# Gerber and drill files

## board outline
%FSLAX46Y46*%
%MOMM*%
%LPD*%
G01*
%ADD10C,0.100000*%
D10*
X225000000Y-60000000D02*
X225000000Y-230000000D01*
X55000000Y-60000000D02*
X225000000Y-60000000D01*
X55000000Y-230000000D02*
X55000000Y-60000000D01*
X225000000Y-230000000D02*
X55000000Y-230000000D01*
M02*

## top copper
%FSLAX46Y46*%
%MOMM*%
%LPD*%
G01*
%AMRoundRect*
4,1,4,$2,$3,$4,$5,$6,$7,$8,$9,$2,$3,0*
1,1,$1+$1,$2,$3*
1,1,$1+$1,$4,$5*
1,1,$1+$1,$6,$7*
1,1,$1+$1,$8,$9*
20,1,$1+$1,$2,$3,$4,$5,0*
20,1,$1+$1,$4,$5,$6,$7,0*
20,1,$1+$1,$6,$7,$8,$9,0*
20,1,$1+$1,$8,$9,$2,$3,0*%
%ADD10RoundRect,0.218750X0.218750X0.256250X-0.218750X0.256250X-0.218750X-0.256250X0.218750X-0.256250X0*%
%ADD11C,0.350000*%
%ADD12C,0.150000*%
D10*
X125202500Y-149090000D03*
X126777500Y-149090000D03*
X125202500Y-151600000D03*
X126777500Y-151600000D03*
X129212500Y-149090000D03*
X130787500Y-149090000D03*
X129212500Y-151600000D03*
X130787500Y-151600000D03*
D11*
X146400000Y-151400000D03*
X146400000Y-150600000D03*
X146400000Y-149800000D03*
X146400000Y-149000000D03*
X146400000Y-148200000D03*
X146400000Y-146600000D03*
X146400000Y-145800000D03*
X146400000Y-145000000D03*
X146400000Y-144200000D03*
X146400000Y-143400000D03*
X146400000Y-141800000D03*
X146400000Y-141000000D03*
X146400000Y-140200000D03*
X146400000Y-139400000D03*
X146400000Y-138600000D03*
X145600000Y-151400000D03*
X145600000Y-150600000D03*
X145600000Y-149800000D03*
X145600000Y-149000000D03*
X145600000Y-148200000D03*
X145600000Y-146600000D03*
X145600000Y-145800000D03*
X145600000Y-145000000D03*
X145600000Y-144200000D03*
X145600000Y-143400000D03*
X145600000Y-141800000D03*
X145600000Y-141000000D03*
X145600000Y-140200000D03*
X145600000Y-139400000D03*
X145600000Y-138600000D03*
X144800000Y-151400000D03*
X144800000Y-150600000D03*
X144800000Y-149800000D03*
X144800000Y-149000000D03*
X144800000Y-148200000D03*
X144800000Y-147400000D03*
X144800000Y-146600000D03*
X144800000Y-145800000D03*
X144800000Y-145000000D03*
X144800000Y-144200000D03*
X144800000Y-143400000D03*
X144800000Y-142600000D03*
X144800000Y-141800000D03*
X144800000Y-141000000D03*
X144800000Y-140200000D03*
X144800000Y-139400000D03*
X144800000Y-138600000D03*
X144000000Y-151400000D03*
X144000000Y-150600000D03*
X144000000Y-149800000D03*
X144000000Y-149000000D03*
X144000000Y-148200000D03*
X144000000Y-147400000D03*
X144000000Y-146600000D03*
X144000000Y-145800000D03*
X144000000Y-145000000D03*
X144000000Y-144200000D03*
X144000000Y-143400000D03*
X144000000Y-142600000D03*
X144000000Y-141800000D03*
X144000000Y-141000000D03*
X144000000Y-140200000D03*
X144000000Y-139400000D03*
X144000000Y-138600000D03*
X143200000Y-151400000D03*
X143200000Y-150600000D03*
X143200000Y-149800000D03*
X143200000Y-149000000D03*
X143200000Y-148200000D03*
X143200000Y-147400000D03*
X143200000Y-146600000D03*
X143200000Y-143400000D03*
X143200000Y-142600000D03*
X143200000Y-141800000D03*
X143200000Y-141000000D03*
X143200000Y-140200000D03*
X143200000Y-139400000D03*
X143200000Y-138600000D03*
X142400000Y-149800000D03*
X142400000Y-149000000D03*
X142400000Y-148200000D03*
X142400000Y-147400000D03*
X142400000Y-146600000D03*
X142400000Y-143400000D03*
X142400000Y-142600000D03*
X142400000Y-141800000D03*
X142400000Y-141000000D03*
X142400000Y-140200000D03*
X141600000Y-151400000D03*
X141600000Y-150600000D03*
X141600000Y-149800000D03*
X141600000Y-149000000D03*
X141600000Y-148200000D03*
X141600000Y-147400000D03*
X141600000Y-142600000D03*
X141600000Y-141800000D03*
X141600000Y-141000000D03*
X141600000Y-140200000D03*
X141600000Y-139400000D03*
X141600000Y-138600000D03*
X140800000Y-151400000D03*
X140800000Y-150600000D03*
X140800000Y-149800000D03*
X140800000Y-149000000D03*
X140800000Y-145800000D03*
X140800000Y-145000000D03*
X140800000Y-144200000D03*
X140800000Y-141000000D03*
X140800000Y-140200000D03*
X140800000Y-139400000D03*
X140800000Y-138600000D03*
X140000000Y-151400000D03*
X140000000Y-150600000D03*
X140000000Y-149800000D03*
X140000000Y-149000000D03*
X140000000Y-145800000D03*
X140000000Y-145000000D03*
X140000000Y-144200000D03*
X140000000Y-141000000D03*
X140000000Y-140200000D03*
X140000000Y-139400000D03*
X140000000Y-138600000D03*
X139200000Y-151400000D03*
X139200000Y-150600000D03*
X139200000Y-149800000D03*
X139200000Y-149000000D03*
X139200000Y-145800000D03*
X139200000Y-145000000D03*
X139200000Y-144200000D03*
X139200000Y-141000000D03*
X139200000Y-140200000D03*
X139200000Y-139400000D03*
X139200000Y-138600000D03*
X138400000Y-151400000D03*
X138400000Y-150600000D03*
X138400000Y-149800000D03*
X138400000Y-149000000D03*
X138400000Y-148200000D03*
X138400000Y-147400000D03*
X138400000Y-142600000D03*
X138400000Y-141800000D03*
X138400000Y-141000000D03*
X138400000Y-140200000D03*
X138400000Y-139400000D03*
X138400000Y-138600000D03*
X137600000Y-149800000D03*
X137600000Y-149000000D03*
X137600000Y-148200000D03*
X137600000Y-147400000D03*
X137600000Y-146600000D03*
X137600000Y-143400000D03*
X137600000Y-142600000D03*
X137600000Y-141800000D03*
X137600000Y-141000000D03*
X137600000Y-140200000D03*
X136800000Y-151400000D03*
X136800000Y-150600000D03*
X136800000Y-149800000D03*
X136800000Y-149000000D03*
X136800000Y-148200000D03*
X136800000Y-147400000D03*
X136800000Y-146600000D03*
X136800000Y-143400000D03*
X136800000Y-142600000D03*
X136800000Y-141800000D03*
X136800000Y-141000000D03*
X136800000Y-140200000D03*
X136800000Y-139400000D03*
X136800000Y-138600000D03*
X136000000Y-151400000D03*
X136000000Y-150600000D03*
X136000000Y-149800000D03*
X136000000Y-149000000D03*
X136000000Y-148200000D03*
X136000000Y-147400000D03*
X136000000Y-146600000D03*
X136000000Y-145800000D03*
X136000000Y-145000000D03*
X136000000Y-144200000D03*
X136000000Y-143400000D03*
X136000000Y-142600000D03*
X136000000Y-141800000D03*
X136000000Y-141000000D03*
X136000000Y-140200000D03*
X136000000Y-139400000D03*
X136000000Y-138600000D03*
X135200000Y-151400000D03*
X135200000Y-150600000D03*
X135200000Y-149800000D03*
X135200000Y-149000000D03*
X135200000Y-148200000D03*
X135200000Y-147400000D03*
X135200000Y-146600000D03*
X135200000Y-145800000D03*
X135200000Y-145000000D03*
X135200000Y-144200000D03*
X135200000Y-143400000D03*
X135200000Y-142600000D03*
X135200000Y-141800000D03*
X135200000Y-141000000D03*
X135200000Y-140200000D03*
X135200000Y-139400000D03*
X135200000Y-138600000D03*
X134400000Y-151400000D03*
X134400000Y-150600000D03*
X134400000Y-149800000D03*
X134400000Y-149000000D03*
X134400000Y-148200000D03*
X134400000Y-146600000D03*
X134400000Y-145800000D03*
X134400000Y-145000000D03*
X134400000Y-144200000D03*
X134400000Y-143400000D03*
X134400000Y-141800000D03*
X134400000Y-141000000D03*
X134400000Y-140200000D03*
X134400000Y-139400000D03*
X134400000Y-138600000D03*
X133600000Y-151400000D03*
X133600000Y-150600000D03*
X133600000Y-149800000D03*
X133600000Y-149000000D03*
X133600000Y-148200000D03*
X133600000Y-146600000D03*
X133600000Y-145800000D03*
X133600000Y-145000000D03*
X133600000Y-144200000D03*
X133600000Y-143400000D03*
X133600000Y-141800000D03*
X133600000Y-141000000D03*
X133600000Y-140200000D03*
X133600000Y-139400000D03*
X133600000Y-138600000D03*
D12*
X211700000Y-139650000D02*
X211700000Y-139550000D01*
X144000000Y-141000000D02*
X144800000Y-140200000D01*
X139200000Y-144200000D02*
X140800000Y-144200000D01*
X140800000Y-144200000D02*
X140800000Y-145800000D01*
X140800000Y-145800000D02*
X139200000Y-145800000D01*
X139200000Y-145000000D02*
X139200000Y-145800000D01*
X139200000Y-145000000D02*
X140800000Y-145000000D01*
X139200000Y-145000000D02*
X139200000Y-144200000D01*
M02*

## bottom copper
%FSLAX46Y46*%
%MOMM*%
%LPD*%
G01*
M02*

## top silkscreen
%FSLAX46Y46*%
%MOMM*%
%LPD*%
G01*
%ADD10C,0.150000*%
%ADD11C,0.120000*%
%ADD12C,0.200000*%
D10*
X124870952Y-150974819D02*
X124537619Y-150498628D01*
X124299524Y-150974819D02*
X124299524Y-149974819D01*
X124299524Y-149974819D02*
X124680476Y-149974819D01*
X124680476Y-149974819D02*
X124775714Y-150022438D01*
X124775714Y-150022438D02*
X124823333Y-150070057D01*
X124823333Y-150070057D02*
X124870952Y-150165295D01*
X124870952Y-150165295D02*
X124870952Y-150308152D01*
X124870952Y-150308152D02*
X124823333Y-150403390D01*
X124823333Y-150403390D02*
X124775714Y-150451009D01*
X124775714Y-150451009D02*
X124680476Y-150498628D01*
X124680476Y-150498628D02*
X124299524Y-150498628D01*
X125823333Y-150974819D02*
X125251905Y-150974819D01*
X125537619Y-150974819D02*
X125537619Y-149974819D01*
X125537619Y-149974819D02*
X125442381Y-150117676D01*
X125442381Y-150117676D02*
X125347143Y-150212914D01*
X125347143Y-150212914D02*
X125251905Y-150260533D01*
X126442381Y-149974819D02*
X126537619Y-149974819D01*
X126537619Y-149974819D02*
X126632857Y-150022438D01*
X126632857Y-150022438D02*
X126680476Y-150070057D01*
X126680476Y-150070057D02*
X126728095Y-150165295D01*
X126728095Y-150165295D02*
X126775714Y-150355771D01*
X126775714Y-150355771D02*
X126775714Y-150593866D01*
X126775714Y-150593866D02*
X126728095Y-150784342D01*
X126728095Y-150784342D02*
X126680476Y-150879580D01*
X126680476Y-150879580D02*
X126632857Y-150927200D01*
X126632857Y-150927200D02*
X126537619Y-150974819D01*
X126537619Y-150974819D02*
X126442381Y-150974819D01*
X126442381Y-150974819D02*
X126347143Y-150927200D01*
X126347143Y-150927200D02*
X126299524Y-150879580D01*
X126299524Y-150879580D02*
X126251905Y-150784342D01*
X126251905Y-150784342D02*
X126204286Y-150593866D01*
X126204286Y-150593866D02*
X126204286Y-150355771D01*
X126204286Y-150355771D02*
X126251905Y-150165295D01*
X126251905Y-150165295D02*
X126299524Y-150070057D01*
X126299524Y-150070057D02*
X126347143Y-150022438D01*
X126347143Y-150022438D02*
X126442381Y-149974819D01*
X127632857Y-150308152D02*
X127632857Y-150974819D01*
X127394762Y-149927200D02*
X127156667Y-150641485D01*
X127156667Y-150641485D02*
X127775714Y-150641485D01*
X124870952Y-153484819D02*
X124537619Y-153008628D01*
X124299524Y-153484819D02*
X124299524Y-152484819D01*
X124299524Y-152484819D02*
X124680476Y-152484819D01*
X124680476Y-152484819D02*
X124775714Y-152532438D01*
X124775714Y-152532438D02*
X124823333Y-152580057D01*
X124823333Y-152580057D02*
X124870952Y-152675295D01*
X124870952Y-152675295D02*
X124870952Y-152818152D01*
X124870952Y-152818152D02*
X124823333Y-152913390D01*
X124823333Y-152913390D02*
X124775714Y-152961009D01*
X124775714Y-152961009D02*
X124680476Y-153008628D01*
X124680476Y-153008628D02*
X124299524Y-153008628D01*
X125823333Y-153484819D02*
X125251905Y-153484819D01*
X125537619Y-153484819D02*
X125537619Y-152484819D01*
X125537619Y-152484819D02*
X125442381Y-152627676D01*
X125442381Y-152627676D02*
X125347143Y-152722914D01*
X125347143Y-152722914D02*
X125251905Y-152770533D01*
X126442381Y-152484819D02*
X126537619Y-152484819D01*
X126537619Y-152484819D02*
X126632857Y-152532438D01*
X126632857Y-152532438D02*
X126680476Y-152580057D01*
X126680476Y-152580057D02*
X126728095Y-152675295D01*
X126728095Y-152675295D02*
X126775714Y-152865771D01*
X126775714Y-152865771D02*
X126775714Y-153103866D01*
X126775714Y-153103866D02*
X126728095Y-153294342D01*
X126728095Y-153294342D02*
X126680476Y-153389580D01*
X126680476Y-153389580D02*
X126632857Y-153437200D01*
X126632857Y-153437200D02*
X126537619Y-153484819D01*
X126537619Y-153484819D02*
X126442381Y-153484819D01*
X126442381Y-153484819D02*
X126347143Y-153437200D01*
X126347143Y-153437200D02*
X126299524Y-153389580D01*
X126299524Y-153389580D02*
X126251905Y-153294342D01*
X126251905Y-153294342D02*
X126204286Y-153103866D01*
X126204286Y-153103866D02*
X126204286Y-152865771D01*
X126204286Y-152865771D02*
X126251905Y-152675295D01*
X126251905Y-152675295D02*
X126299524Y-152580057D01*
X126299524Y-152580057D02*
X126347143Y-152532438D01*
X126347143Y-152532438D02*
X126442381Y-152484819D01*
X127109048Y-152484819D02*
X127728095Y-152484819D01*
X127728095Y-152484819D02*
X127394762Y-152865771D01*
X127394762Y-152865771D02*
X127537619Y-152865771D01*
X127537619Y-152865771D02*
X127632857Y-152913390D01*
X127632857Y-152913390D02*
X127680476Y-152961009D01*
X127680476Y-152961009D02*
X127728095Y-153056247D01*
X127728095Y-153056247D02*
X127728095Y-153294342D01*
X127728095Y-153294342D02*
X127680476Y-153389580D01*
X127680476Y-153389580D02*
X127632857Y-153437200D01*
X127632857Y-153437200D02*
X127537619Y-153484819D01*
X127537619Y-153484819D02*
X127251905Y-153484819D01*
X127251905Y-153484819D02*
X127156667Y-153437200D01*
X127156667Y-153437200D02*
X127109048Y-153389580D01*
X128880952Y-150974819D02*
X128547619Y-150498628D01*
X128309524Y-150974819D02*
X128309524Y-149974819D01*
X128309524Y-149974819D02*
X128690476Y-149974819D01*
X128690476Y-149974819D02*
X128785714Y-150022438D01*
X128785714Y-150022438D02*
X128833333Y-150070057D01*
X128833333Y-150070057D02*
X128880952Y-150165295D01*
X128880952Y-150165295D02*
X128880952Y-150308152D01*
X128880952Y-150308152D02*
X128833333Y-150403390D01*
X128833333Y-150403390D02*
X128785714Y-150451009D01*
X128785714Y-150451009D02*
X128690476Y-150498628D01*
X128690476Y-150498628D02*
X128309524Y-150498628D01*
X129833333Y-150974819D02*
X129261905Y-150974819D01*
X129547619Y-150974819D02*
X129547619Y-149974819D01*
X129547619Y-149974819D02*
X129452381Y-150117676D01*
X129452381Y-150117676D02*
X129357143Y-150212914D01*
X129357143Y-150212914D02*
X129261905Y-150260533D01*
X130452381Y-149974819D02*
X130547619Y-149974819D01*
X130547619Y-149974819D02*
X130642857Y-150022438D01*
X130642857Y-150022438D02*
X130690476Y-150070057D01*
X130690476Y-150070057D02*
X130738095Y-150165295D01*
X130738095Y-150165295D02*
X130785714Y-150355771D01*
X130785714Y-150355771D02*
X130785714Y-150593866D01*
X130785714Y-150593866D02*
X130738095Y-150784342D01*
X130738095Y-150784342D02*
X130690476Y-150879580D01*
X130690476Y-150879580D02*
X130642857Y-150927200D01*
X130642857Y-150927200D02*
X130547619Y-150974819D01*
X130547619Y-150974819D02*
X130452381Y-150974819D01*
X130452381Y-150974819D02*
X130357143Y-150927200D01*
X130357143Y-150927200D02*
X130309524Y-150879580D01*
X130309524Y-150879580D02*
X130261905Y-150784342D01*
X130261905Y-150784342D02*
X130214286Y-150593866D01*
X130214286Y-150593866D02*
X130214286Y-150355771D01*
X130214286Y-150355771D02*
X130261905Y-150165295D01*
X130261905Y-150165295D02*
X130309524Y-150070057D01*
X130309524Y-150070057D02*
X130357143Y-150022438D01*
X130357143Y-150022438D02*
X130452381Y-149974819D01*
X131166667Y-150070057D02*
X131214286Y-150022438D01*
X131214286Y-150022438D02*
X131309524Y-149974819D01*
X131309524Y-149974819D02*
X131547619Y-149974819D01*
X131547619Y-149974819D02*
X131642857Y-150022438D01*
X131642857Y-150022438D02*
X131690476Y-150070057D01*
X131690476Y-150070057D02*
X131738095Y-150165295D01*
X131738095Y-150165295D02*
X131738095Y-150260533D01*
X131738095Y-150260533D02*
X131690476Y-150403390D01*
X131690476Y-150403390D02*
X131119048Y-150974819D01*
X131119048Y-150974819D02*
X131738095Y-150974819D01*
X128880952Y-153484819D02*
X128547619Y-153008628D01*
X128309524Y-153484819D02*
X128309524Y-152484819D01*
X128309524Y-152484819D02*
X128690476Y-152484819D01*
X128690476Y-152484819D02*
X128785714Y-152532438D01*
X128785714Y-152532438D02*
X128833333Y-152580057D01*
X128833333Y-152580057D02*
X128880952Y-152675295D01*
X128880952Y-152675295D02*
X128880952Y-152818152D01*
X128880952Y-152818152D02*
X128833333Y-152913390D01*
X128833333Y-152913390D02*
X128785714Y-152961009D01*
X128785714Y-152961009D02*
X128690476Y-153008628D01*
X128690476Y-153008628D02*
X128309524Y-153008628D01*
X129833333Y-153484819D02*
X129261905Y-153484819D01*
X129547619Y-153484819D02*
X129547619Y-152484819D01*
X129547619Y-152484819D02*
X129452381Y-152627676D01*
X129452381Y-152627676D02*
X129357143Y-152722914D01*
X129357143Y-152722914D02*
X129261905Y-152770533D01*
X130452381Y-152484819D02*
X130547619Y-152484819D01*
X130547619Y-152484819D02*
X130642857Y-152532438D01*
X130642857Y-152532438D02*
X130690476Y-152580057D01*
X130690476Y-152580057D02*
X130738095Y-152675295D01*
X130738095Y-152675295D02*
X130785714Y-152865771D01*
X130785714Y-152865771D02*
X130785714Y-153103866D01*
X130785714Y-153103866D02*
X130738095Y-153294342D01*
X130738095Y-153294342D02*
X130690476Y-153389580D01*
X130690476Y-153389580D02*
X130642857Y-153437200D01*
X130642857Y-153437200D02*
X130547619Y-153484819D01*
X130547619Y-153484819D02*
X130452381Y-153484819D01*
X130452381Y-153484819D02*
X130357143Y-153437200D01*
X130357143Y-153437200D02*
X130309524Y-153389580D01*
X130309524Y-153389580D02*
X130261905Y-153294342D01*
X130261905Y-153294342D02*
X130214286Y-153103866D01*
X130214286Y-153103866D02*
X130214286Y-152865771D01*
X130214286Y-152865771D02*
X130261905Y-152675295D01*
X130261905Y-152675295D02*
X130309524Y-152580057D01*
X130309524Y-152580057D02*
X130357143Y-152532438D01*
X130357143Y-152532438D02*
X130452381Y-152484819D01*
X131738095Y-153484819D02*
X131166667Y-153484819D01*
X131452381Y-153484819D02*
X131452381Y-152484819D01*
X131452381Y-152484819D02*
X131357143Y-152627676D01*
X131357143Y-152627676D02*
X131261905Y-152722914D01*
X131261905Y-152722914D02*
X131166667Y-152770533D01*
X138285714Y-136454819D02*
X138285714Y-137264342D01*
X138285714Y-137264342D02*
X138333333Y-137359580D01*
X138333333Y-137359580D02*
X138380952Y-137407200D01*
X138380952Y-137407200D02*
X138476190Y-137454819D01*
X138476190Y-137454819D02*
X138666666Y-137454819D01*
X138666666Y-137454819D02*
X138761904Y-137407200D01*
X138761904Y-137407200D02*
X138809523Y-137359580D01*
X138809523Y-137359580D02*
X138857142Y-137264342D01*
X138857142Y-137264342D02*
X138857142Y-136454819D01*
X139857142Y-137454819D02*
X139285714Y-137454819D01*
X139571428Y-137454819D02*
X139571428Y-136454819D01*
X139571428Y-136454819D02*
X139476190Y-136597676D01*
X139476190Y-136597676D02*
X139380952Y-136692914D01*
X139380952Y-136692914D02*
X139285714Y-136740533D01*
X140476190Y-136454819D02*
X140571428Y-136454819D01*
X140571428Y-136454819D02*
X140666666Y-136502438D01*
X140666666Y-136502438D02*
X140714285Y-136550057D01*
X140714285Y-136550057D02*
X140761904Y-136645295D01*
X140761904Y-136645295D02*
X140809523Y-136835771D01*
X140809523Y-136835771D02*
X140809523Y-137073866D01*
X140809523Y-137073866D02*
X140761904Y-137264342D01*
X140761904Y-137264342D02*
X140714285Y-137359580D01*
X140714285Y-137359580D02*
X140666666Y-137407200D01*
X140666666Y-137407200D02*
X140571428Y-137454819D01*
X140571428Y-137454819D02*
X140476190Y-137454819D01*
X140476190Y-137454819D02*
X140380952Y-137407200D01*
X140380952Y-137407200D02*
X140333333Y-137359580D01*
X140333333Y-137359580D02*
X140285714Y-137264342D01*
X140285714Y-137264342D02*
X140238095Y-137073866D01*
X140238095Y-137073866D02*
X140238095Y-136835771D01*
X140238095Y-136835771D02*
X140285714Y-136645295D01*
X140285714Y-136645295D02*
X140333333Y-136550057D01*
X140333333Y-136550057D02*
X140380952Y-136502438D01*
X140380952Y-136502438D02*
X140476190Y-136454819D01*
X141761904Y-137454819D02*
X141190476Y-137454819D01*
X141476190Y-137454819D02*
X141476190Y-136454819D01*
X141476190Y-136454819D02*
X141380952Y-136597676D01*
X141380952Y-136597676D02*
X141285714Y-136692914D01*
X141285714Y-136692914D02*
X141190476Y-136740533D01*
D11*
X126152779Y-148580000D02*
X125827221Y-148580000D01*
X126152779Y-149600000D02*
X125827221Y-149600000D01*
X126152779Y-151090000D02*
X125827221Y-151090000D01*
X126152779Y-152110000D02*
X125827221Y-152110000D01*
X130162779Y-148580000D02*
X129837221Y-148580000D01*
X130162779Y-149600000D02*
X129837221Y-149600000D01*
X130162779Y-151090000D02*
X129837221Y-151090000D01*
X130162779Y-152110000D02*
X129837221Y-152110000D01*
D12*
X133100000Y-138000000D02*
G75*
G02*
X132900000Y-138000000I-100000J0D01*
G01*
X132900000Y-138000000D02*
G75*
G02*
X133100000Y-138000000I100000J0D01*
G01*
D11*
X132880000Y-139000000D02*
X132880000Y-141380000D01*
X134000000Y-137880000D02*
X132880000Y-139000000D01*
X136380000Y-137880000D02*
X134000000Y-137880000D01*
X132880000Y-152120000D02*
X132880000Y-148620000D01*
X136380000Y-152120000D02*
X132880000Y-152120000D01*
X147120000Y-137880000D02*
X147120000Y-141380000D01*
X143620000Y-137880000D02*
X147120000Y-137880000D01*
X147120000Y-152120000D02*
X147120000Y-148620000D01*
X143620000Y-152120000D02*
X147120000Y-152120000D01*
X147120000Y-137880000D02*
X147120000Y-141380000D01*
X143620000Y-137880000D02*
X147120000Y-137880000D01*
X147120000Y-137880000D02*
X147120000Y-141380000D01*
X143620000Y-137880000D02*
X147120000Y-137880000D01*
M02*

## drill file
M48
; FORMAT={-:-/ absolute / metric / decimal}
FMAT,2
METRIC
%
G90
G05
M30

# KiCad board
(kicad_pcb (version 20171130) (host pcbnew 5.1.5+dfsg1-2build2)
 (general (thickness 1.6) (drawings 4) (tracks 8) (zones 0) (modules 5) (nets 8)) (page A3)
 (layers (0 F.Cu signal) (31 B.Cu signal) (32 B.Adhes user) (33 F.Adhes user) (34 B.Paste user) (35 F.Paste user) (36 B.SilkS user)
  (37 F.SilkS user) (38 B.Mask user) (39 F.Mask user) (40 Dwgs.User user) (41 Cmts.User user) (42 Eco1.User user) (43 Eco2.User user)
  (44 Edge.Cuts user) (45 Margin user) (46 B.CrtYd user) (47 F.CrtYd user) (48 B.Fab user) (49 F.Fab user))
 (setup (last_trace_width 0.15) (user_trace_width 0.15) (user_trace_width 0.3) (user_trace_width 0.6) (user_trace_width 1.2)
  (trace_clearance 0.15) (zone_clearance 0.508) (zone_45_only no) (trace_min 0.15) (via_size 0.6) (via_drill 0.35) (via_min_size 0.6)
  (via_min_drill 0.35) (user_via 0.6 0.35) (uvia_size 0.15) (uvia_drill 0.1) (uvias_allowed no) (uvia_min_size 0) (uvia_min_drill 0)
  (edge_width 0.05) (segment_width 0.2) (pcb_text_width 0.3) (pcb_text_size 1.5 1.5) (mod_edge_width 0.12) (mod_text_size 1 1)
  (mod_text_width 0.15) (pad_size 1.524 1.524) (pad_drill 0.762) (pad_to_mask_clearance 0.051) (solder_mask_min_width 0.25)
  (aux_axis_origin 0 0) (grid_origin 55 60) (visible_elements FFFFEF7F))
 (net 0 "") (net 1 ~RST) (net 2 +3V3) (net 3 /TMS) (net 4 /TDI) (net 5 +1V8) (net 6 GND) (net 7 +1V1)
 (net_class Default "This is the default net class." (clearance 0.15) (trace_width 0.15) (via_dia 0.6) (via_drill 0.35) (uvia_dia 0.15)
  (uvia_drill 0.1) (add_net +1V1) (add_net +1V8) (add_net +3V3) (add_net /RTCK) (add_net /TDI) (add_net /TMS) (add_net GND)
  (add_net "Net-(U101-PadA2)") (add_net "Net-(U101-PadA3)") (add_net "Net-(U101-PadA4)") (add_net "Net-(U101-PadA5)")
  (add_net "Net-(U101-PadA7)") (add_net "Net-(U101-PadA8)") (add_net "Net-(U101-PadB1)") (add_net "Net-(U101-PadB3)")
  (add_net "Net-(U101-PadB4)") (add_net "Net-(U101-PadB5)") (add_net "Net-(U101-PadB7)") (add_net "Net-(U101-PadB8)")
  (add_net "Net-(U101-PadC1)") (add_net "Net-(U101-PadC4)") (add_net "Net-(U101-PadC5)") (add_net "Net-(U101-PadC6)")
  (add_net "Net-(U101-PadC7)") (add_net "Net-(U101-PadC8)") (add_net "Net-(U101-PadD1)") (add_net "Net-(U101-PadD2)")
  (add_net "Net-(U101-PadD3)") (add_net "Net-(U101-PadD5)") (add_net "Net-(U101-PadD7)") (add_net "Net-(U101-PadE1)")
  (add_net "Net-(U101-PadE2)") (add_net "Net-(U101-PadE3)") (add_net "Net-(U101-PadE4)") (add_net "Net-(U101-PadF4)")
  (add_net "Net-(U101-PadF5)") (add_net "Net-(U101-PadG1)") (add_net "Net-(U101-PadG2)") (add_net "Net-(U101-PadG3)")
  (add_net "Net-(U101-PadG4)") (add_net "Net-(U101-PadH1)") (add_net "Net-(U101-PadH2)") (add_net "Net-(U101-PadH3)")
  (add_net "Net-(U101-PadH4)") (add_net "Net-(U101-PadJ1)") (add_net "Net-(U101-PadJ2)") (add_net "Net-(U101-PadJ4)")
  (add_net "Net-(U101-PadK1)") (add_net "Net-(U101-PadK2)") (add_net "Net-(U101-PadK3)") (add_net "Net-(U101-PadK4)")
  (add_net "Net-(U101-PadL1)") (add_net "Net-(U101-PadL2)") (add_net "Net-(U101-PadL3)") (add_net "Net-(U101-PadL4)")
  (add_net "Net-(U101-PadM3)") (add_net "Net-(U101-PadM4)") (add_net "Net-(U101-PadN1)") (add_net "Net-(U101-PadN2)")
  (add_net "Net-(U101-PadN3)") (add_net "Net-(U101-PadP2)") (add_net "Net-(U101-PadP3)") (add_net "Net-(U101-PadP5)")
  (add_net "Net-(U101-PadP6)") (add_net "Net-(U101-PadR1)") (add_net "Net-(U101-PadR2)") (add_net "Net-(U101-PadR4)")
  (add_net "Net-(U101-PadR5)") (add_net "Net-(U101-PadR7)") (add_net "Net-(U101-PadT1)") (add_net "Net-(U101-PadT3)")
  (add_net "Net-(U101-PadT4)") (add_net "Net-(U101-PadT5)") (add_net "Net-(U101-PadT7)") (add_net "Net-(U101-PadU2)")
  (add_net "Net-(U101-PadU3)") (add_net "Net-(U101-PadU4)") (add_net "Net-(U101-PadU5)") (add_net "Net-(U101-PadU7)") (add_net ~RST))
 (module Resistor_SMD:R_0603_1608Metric (layer F.Cu) (at 125.99 149.09 180)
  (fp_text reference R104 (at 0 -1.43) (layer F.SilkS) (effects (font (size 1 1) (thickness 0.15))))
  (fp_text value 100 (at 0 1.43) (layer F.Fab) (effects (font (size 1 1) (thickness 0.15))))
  (fp_line (start -0.162779 0.51) (end 0.162779 0.51) (layer F.SilkS) (width 0.12))
  (fp_line (start -0.162779 -0.51) (end 0.162779 -0.51) (layer F.SilkS) (width 0.12))
  (pad 2 smd roundrect (at 0.7875 0 180) (size 0.875 0.95) (layers F.Cu F.Paste F.Mask) (roundrect_rratio 0.25))
  (pad 1 smd roundrect (at -0.7875 0 180) (size 0.875 0.95) (layers F.Cu F.Paste F.Mask) (roundrect_rratio 0.25) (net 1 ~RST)))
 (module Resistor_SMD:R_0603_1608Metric (layer F.Cu) (at 125.99 151.6 180)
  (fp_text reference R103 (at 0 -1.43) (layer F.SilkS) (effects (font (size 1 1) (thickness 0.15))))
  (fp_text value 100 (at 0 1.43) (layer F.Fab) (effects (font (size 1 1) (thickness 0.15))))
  (fp_line (start -0.162779 0.51) (end 0.162779 0.51) (layer F.SilkS) (width 0.12))
  (fp_line (start -0.162779 -0.51) (end 0.162779 -0.51) (layer F.SilkS) (width 0.12))
  (pad 2 smd roundrect (at 0.7875 0 180) (size 0.875 0.95) (layers F.Cu F.Paste F.Mask) (roundrect_rratio 0.25) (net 1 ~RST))
  (pad 1 smd roundrect (at -0.7875 0 180) (size 0.875 0.95) (layers F.Cu F.Paste F.Mask) (roundrect_rratio 0.25) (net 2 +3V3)))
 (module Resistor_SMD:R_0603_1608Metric (layer F.Cu) (at 130 149.09 180)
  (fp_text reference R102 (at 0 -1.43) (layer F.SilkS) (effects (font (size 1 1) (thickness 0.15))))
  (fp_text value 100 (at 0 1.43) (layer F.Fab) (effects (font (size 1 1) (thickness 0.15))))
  (fp_line (start -0.162779 0.51) (end 0.162779 0.51) (layer F.SilkS) (width 0.12))
  (fp_line (start -0.162779 -0.51) (end 0.162779 -0.51) (layer F.SilkS) (width 0.12))
  (pad 2 smd roundrect (at 0.7875 0 180) (size 0.875 0.95) (layers F.Cu F.Paste F.Mask) (roundrect_rratio 0.25) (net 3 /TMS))
  (pad 1 smd roundrect (at -0.7875 0 180) (size 0.875 0.95) (layers F.Cu F.Paste F.Mask) (roundrect_rratio 0.25) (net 2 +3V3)))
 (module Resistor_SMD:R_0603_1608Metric (layer F.Cu) (at 130 151.6 180)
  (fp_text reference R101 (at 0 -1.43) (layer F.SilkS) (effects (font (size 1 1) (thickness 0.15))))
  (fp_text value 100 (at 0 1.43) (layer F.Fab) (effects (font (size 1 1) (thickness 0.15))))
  (fp_line (start -0.162779 0.51) (end 0.162779 0.51) (layer F.SilkS) (width 0.12))
  (fp_line (start -0.162779 -0.51) (end 0.162779 -0.51) (layer F.SilkS) (width 0.12))
  (pad 2 smd roundrect (at 0.7875 0 180) (size 0.875 0.95) (layers F.Cu F.Paste F.Mask) (roundrect_rratio 0.25) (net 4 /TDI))
  (pad 1 smd roundrect (at -0.7875 0 180) (size 0.875 0.95) (layers F.Cu F.Paste F.Mask) (roundrect_rratio 0.25) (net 2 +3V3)))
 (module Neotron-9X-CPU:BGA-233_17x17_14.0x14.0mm (layer F.Cu) (at 140 145)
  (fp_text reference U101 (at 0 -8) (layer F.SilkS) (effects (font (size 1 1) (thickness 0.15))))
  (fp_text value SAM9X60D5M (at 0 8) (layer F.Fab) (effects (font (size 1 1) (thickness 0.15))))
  (fp_circle (center -7 -7) (end -7 -6.9) (layer F.SilkS) (width 0.2))
  (fp_line (start -7.12 -6) (end -7.12 -3.62) (layer F.SilkS) (width 0.12))
  (fp_line (start -6 -7.12) (end -7.12 -6) (layer F.SilkS) (width 0.12))
  (fp_line (start -3.62 -7.12) (end -6 -7.12) (layer F.SilkS) (width 0.12))
  (fp_line (start -7.12 7.12) (end -7.12 3.62) (layer F.SilkS) (width 0.12))
  (fp_line (start -3.62 7.12) (end -7.12 7.12) (layer F.SilkS) (width 0.12))
  (fp_line (start 7.12 -7.12) (end 7.12 -3.62) (layer F.SilkS) (width 0.12))
  (fp_line (start 3.62 -7.12) (end 7.12 -7.12) (layer F.SilkS) (width 0.12))
  (fp_line (start 7.12 7.12) (end 7.12 3.62) (layer F.SilkS) (width 0.12))
  (fp_line (start 3.62 7.12) (end 7.12 7.12) (layer F.SilkS) (width 0.12))
  (fp_line (start 7.12 -7.12) (end 7.12 -3.62) (layer F.SilkS) (width 0.12))
  (fp_line (start 3.62 -7.12) (end 7.12 -7.12) (layer F.SilkS) (width 0.12))
  (fp_line (start 7.12 -7.12) (end 7.12 -3.62) (layer F.SilkS) (width 0.12))
  (fp_line (start 3.62 -7.12) (end 7.12 -7.12) (layer F.SilkS) (width 0.12))
  (pad U17 smd circle (at 6.4 6.4) (size 0.35 0.35) (layers F.Cu F.Paste F.Mask))
  (pad T17 smd circle (at 6.4 5.6) (size 0.35 0.35) (layers F.Cu F.Paste F.Mask))
  (pad R17 smd circle (at 6.4 4.8) (size 0.35 0.35) (layers F.Cu F.Paste F.Mask))
  (pad P17 smd circle (at 6.4 4) (size 0.35 0.35) (layers F.Cu F.Paste F.Mask))
  (pad N17 smd circle (at 6.4 3.2) (size 0.35 0.35) (layers F.Cu F.Paste F.Mask))
  (pad L17 smd circle (at 6.4 1.6) (size 0.35 0.35) (layers F.Cu F.Paste F.Mask))
  (pad K17 smd circle (at 6.4 0.8) (size 0.35 0.35) (layers F.Cu F.Paste F.Mask))
  (pad J17 smd circle (at 6.4 0) (size 0.35 0.35) (layers F.Cu F.Paste F.Mask))
  (pad H17 smd circle (at 6.4 -0.8) (size 0.35 0.35) (layers F.Cu F.Paste F.Mask))
  (pad G17 smd circle (at 6.4 -1.6) (size 0.35 0.35) (layers F.Cu F.Paste F.Mask))
  (pad E17 smd circle (at 6.4 -3.2) (size 0.35 0.35) (layers F.Cu F.Paste F.Mask))
  (pad D17 smd circle (at 6.4 -4) (size 0.35 0.35) (layers F.Cu F.Paste F.Mask))
  (pad C17 smd circle (at 6.4 -4.8) (size 0.35 0.35) (layers F.Cu F.Paste F.Mask))
  (pad B17 smd circle (at 6.4 -5.6) (size 0.35 0.35) (layers F.Cu F.Paste F.Mask) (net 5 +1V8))
  (pad A17 smd circle (at 6.4 -6.4) (size 0.35 0.35) (layers F.Cu F.Paste F.Mask) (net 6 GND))
  (pad U16 smd circle (at 5.6 6.4) (size 0.35 0.35) (layers F.Cu F.Paste F.Mask))
  (pad T16 smd circle (at 5.6 5.6) (size 0.35 0.35) (layers F.Cu F.Paste F.Mask) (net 6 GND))
  (pad R16 smd circle (at 5.6 4.8) (size 0.35 0.35) (layers F.Cu F.Paste F.Mask) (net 6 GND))
  (pad P16 smd circle (at 5.6 4) (size 0.35 0.35) (layers F.Cu F.Paste F.Mask))
  (pad N16 smd circle (at 5.6 3.2) (size 0.35 0.35) (layers F.Cu F.Paste F.Mask) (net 3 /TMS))
  (pad L16 smd circle (at 5.6 1.6) (size 0.35 0.35) (layers F.Cu F.Paste F.Mask))
  (pad K16 smd circle (at 5.6 0.8) (size 0.35 0.35) (layers F.Cu F.Paste F.Mask))
  (pad J16 smd circle (at 5.6 0) (size 0.35 0.35) (layers F.Cu F.Paste F.Mask))
  (pad H16 smd circle (at 5.6 -0.8) (size 0.35 0.35) (layers F.Cu F.Paste F.Mask))
  (pad G16 smd circle (at 5.6 -1.6) (size 0.35 0.35) (layers F.Cu F.Paste F.Mask))
  (pad E16 smd circle (at 5.6 -3.2) (size 0.35 0.35) (layers F.Cu F.Paste F.Mask))
  (pad D16 smd circle (at 5.6 -4) (size 0.35 0.35) (layers F.Cu F.Paste F.Mask))
  (pad C16 smd circle (at 5.6 -4.8) (size 0.35 0.35) (layers F.Cu F.Paste F.Mask) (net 5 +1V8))
  (pad B16 smd circle (at 5.6 -5.6) (size 0.35 0.35) (layers F.Cu F.Paste F.Mask) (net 6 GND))
  (pad A16 smd circle (at 5.6 -6.4) (size 0.35 0.35) (layers F.Cu F.Paste F.Mask) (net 5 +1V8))
  (pad U15 smd circle (at 4.8 6.4) (size 0.35 0.35) (layers F.Cu F.Paste F.Mask) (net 6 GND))
  (pad T15 smd circle (at 4.8 5.6) (size 0.35 0.35) (layers F.Cu F.Paste F.Mask))
  (pad R15 smd circle (at 4.8 4.8) (size 0.35 0.35) (layers F.Cu F.Paste F.Mask) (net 6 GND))
  (pad P15 smd circle (at 4.8 4) (size 0.35 0.35) (layers F.Cu F.Paste F.Mask))
  (pad N15 smd circle (at 4.8 3.2) (size 0.35 0.35) (layers F.Cu F.Paste F.Mask))
  (pad M15 smd circle (at 4.8 2.4) (size 0.35 0.35) (layers F.Cu F.Paste F.Mask))
  (pad L15 smd circle (at 4.8 1.6) (size 0.35 0.35) (layers F.Cu F.Paste F.Mask) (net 4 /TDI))
  (pad K15 smd circle (at 4.8 0.8) (size 0.35 0.35) (layers F.Cu F.Paste F.Mask))
  (pad J15 smd circle (at 4.8 0) (size 0.35 0.35) (layers F.Cu F.Paste F.Mask) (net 6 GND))
  (pad H15 smd circle (at 4.8 -0.8) (size 0.35 0.35) (layers F.Cu F.Paste F.Mask))
  (pad G15 smd circle (at 4.8 -1.6) (size 0.35 0.35) (layers F.Cu F.Paste F.Mask))
  (pad F15 smd circle (at 4.8 -2.4) (size 0.35 0.35) (layers F.Cu F.Paste F.Mask) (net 6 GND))
  (pad E15 smd circle (at 4.8 -3.2) (size 0.35 0.35) (layers F.Cu F.Paste F.Mask))
  (pad D15 smd circle (at 4.8 -4) (size 0.35 0.35) (layers F.Cu F.Paste F.Mask) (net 5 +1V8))
  (pad C15 smd circle (at 4.8 -4.8) (size 0.35 0.35) (layers F.Cu F.Paste F.Mask) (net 6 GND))
  (pad B15 smd circle (at 4.8 -5.6) (size 0.35 0.35) (layers F.Cu F.Paste F.Mask) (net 5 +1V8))
  (pad A15 smd circle (at 4.8 -6.4) (size 0.35 0.35) (layers F.Cu F.Paste F.Mask) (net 6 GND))
  (pad U14 smd circle (at 4 6.4) (size 0.35 0.35) (layers F.Cu F.Paste F.Mask))
  (pad T14 smd circle (at 4 5.6) (size 0.35 0.35) (layers F.Cu F.Paste F.Mask))
  (pad R14 smd circle (at 4 4.8) (size 0.35 0.35) (layers F.Cu F.Paste F.Mask))
  (pad P14 smd circle (at 4 4) (size 0.35 0.35) (layers F.Cu F.Paste F.Mask) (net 6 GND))
  (pad N14 smd circle (at 4 3.2) (size 0.35 0.35) (layers F.Cu F.Paste F.Mask))
  (pad M14 smd circle (at 4 2.4) (size 0.35 0.35) (layers F.Cu F.Paste F.Mask) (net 6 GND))
  (pad L14 smd circle (at 4 1.6) (size 0.35 0.35) (layers F.Cu F.Paste F.Mask) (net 6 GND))
  (pad K14 smd circle (at 4 0.8) (size 0.35 0.35) (layers F.Cu F.Paste F.Mask))
  (pad J14 smd circle (at 4 0) (size 0.35 0.35) (layers F.Cu F.Paste F.Mask))
  (pad H14 smd circle (at 4 -0.8) (size 0.35 0.35) (layers F.Cu F.Paste F.Mask))
  (pad G14 smd circle (at 4 -1.6) (size 0.35 0.35) (layers F.Cu F.Paste F.Mask))
  (pad F14 smd circle (at 4 -2.4) (size 0.35 0.35) (layers F.Cu F.Paste F.Mask))
  (pad E14 smd circle (at 4 -3.2) (size 0.35 0.35) (layers F.Cu F.Paste F.Mask))
  (pad D14 smd circle (at 4 -4) (size 0.35 0.35) (layers F.Cu F.Paste F.Mask) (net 6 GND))
  (pad C14 smd circle (at 4 -4.8) (size 0.35 0.35) (layers F.Cu F.Paste F.Mask) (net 5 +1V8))
  (pad B14 smd circle (at 4 -5.6) (size 0.35 0.35) (layers F.Cu F.Paste F.Mask) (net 6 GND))
  (pad A14 smd circle (at 4 -6.4) (size 0.35 0.35) (layers F.Cu F.Paste F.Mask))
  (pad U13 smd circle (at 3.2 6.4) (size 0.35 0.35) (layers F.Cu F.Paste F.Mask))
  (pad T13 smd circle (at 3.2 5.6) (size 0.35 0.35) (layers F.Cu F.Paste F.Mask))
  (pad R13 smd circle (at 3.2 4.8) (size 0.35 0.35) (layers F.Cu F.Paste F.Mask))
  (pad P13 smd circle (at 3.2 4) (size 0.35 0.35) (layers F.Cu F.Paste F.Mask))
  (pad N13 smd circle (at 3.2 3.2) (size 0.35 0.35) (layers F.Cu F.Paste F.Mask) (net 6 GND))
  (pad M13 smd circle (at 3.2 2.4) (size 0.35 0.35) (layers F.Cu F.Paste F.Mask) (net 6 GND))
  (pad L13 smd circle (at 3.2 1.6) (size 0.35 0.35) (layers F.Cu F.Paste F.Mask) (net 6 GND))
  (pad G13 smd circle (at 3.2 -1.6) (size 0.35 0.35) (layers F.Cu F.Paste F.Mask) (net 5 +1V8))
  (pad F13 smd circle (at 3.2 -2.4) (size 0.35 0.35) (layers F.Cu F.Paste F.Mask) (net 5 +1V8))
  (pad E13 smd circle (at 3.2 -3.2) (size 0.35 0.35) (layers F.Cu F.Paste F.Mask) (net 6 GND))
  (pad D13 smd circle (at 3.2 -4) (size 0.35 0.35) (layers F.Cu F.Paste F.Mask) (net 5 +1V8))
  (pad C13 smd circle (at 3.2 -4.8) (size 0.35 0.35) (layers F.Cu F.Paste F.Mask) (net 6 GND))
  (pad B13 smd circle (at 3.2 -5.6) (size 0.35 0.35) (layers F.Cu F.Paste F.Mask) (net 6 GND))
  (pad A13 smd circle (at 3.2 -6.4) (size 0.35 0.35) (layers F.Cu F.Paste F.Mask) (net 6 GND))
  (pad R12 smd circle (at 2.4 4.8) (size 0.35 0.35) (layers F.Cu F.Paste F.Mask))
  (pad P12 smd circle (at 2.4 4) (size 0.35 0.35) (layers F.Cu F.Paste F.Mask))
  (pad N12 smd circle (at 2.4 3.2) (size 0.35 0.35) (layers F.Cu F.Paste F.Mask) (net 6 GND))
  (pad M12 smd circle (at 2.4 2.4) (size 0.35 0.35) (layers F.Cu F.Paste F.Mask) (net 6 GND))
  (pad L12 smd circle (at 2.4 1.6) (size 0.35 0.35) (layers F.Cu F.Paste F.Mask) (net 6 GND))
  (pad G12 smd circle (at 2.4 -1.6) (size 0.35 0.35) (layers F.Cu F.Paste F.Mask) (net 6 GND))
  (pad F12 smd circle (at 2.4 -2.4) (size 0.35 0.35) (layers F.Cu F.Paste F.Mask) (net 6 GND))
  (pad E12 smd circle (at 2.4 -3.2) (size 0.35 0.35) (layers F.Cu F.Paste F.Mask) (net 5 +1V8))
  (pad D12 smd circle (at 2.4 -4) (size 0.35 0.35) (layers F.Cu F.Paste F.Mask))
  (pad C12 smd circle (at 2.4 -4.8) (size 0.35 0.35) (layers F.Cu F.Paste F.Mask) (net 6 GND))
  (pad U11 smd circle (at 1.6 6.4) (size 0.35 0.35) (layers F.Cu F.Paste F.Mask))
  (pad T11 smd circle (at 1.6 5.6) (size 0.35 0.35) (layers F.Cu F.Paste F.Mask))
  (pad R11 smd circle (at 1.6 4.8) (size 0.35 0.35) (layers F.Cu F.Paste F.Mask) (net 6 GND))
  (pad P11 smd circle (at 1.6 4) (size 0.35 0.35) (layers F.Cu F.Paste F.Mask))
  (pad N11 smd circle (at 1.6 3.2) (size 0.35 0.35) (layers F.Cu F.Paste F.Mask))
  (pad M11 smd circle (at 1.6 2.4) (size 0.35 0.35) (layers F.Cu F.Paste F.Mask) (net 6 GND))
  (pad F11 smd circle (at 1.6 -2.4) (size 0.35 0.35) (layers F.Cu F.Paste F.Mask) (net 6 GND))
  (pad E11 smd circle (at 1.6 -3.2) (size 0.35 0.35) (layers F.Cu F.Paste F.Mask) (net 5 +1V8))
  (pad D11 smd circle (at 1.6 -4) (size 0.35 0.35) (layers F.Cu F.Paste F.Mask))
  (pad C11 smd circle (at 1.6 -4.8) (size 0.35 0.35) (layers F.Cu F.Paste F.Mask))
  (pad B11 smd circle (at 1.6 -5.6) (size 0.35 0.35) (layers F.Cu F.Paste F.Mask))
  (pad A11 smd circle (at 1.6 -6.4) (size 0.35 0.35) (layers F.Cu F.Paste F.Mask))
  (pad U10 smd circle (at 0.8 6.4) (size 0.35 0.35) (layers F.Cu F.Paste F.Mask))
  (pad T10 smd circle (at 0.8 5.6) (size 0.35 0.35) (layers F.Cu F.Paste F.Mask))
  (pad R10 smd circle (at 0.8 4.8) (size 0.35 0.35) (layers F.Cu F.Paste F.Mask))
  (pad P10 smd circle (at 0.8 4) (size 0.35 0.35) (layers F.Cu F.Paste F.Mask) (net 6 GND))
  (pad K10 smd circle (at 0.8 0.8) (size 0.35 0.35) (layers F.Cu F.Paste F.Mask) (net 6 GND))
  (pad J10 smd circle (at 0.8 0) (size 0.35 0.35) (layers F.Cu F.Paste F.Mask) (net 6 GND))
  (pad H10 smd circle (at 0.8 -0.8) (size 0.35 0.35) (layers F.Cu F.Paste F.Mask) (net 6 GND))
  (pad D10 smd circle (at 0.8 -4) (size 0.35 0.35) (layers F.Cu F.Paste F.Mask))
  (pad C10 smd circle (at 0.8 -4.8) (size 0.35 0.35) (layers F.Cu F.Paste F.Mask))
  (pad B10 smd circle (at 0.8 -5.6) (size 0.35 0.35) (layers F.Cu F.Paste F.Mask))
  (pad A10 smd circle (at 0.8 -6.4) (size 0.35 0.35) (layers F.Cu F.Paste F.Mask))
  (pad U9 smd circle (at 0 6.4) (size 0.35 0.35) (layers F.Cu F.Paste F.Mask))
  (pad T9 smd circle (at 0 5.6) (size 0.35 0.35) (layers F.Cu F.Paste F.Mask))
  (pad R9 smd circle (at 0 4.8) (size 0.35 0.35) (layers F.Cu F.Paste F.Mask) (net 6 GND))
  (pad P9 smd circle (at 0 4) (size 0.35 0.35) (layers F.Cu F.Paste F.Mask))
  (pad K9 smd circle (at 0 0.8) (size 0.35 0.35) (layers F.Cu F.Paste F.Mask) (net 6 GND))
  (pad J9 smd circle (at 0 0) (size 0.35 0.35) (layers F.Cu F.Paste F.Mask) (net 6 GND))
  (pad H9 smd circle (at 0 -0.8) (size 0.35 0.35) (layers F.Cu F.Paste F.Mask) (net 6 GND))
  (pad D9 smd circle (at 0 -4) (size 0.35 0.35) (layers F.Cu F.Paste F.Mask))
  (pad C9 smd circle (at 0 -4.8) (size 0.35 0.35) (layers F.Cu F.Paste F.Mask) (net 6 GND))
  (pad B9 smd circle (at 0 -5.6) (size 0.35 0.35) (layers F.Cu F.Paste F.Mask))
  (pad A9 smd circle (at 0 -6.4) (size 0.35 0.35) (layers F.Cu F.Paste F.Mask))
  (pad U8 smd circle (at -0.8 6.4) (size 0.35 0.35) (layers F.Cu F.Paste F.Mask))
  (pad T8 smd circle (at -0.8 5.6) (size 0.35 0.35) (layers F.Cu F.Paste F.Mask))
  (pad R8 smd circle (at -0.8 4.8) (size 0.35 0.35) (layers F.Cu F.Paste F.Mask))
  (pad P8 smd circle (at -0.8 4) (size 0.35 0.35) (layers F.Cu F.Paste F.Mask))
  (pad K8 smd circle (at -0.8 0.8) (size 0.35 0.35) (layers F.Cu F.Paste F.Mask) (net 6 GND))
  (pad J8 smd circle (at -0.8 0) (size 0.35 0.35) (layers F.Cu F.Paste F.Mask) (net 6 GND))
  (pad H8 smd circle (at -0.8 -0.8) (size 0.35 0.35) (layers F.Cu F.Paste F.Mask) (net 6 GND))
  (pad D8 smd circle (at -0.8 -4) (size 0.35 0.35) (layers F.Cu F.Paste F.Mask) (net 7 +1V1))
  (pad C8 smd circle (at -0.8 -4.8) (size 0.35 0.35) (layers F.Cu F.Paste F.Mask))
  (pad B8 smd circle (at -0.8 -5.6) (size 0.35 0.35) (layers F.Cu F.Paste F.Mask))
  (pad A8 smd circle (at -0.8 -6.4) (size 0.35 0.35) (layers F.Cu F.Paste F.Mask))
  (pad U7 smd circle (at -1.6 6.4) (size 0.35 0.35) (layers F.Cu F.Paste F.Mask))
  (pad T7 smd circle (at -1.6 5.6) (size 0.35 0.35) (layers F.Cu F.Paste F.Mask))
  (pad R7 smd circle (at -1.6 4.8) (size 0.35 0.35) (layers F.Cu F.Paste F.Mask))
  (pad P7 smd circle (at -1.6 4) (size 0.35 0.35) (layers F.Cu F.Paste F.Mask) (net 6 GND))
  (pad N7 smd circle (at -1.6 3.2) (size 0.35 0.35) (layers F.Cu F.Paste F.Mask) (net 6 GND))
  (pad M7 smd circle (at -1.6 2.4) (size 0.35 0.35) (layers F.Cu F.Paste F.Mask) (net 7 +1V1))
  (pad F7 smd circle (at -1.6 -2.4) (size 0.35 0.35) (layers F.Cu F.Paste F.Mask) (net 6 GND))
  (pad E7 smd circle (at -1.6 -3.2) (size 0.35 0.35) (layers F.Cu F.Paste F.Mask) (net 6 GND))
  (pad D7 smd circle (at -1.6 -4) (size 0.35 0.35) (layers F.Cu F.Paste F.Mask))
  (pad C7 smd circle (at -1.6 -4.8) (size 0.35 0.35) (layers F.Cu F.Paste F.Mask))
  (pad B7 smd circle (at -1.6 -5.6) (size 0.35 0.35) (layers F.Cu F.Paste F.Mask))
  (pad A7 smd circle (at -1.6 -6.4) (size 0.35 0.35) (layers F.Cu F.Paste F.Mask))
  (pad R6 smd circle (at -2.4 4.8) (size 0.35 0.35) (layers F.Cu F.Paste F.Mask) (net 7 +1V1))
  (pad P6 smd circle (at -2.4 4) (size 0.35 0.35) (layers F.Cu F.Paste F.Mask))
  (pad N6 smd circle (at -2.4 3.2) (size 0.35 0.35) (layers F.Cu F.Paste F.Mask) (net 6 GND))
  (pad M6 smd circle (at -2.4 2.4) (size 0.35 0.35) (layers F.Cu F.Paste F.Mask) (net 6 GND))
  (pad L6 smd circle (at -2.4 1.6) (size 0.35 0.35) (layers F.Cu F.Paste F.Mask) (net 7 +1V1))
  (pad G6 smd circle (at -2.4 -1.6) (size 0.35 0.35) (layers F.Cu F.Paste F.Mask) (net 6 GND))
  (pad F6 smd circle (at -2.4 -2.4) (size 0.35 0.35) (layers F.Cu F.Paste F.Mask) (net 6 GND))
  (pad E6 smd circle (at -2.4 -3.2) (size 0.35 0.35) (layers F.Cu F.Paste F.Mask) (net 6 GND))
  (pad D6 smd circle (at -2.4 -4) (size 0.35 0.35) (layers F.Cu F.Paste F.Mask) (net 7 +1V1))
  (pad C6 smd circle (at -2.4 -4.8) (size 0.35 0.35) (layers F.Cu F.Paste F.Mask))
  (pad U5 smd circle (at -3.2 6.4) (size 0.35 0.35) (layers F.Cu F.Paste F.Mask))
  (pad T5 smd circle (at -3.2 5.6) (size 0.35 0.35) (layers F.Cu F.Paste F.Mask))
  (pad R5 smd circle (at -3.2 4.8) (size 0.35 0.35) (layers F.Cu F.Paste F.Mask))
  (pad P5 smd circle (at -3.2 4) (size 0.35 0.35) (layers F.Cu F.Paste F.Mask))
  (pad N5 smd circle (at -3.2 3.2) (size 0.35 0.35) (layers F.Cu F.Paste F.Mask) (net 6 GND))
  (pad M5 smd circle (at -3.2 2.4) (size 0.35 0.35) (layers F.Cu F.Paste F.Mask) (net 6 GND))
  (pad L5 smd circle (at -3.2 1.6) (size 0.35 0.35) (layers F.Cu F.Paste F.Mask) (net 6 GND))
  (pad G5 smd circle (at -3.2 -1.6) (size 0.35 0.35) (layers F.Cu F.Paste F.Mask) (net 7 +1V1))
  (pad F5 smd circle (at -3.2 -2.4) (size 0.35 0.35) (layers F.Cu F.Paste F.Mask))
  (pad E5 smd circle (at -3.2 -3.2) (size 0.35 0.35) (layers F.Cu F.Paste F.Mask) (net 6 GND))
  (pad D5 smd circle (at -3.2 -4) (size 0.35 0.35) (layers F.Cu F.Paste F.Mask))
  (pad C5 smd circle (at -3.2 -4.8) (size 0.35 0.35) (layers F.Cu F.Paste F.Mask))
  (pad B5 smd circle (at -3.2 -5.6) (size 0.35 0.35) (layers F.Cu F.Paste F.Mask))
  (pad A5 smd circle (at -3.2 -6.4) (size 0.35 0.35) (layers F.Cu F.Paste F.Mask))
  (pad U4 smd circle (at -4 6.4) (size 0.35 0.35) (layers F.Cu F.Paste F.Mask))
  (pad T4 smd circle (at -4 5.6) (size 0.35 0.35) (layers F.Cu F.Paste F.Mask))
  (pad R4 smd circle (at -4 4.8) (size 0.35 0.35) (layers F.Cu F.Paste F.Mask))
  (pad P4 smd circle (at -4 4) (size 0.35 0.35) (layers F.Cu F.Paste F.Mask) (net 6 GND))
  (pad N4 smd circle (at -4 3.2) (size 0.35 0.35) (layers F.Cu F.Paste F.Mask))
  (pad M4 smd circle (at -4 2.4) (size 0.35 0.35) (layers F.Cu F.Paste F.Mask))
  (pad L4 smd circle (at -4 1.6) (size 0.35 0.35) (layers F.Cu F.Paste F.Mask))
  (pad K4 smd circle (at -4 0.8) (size 0.35 0.35) (layers F.Cu F.Paste F.Mask))
  (pad J4 smd circle (at -4 0) (size 0.35 0.35) (layers F.Cu F.Paste F.Mask))
  (pad H4 smd circle (at -4 -0.8) (size 0.35 0.35) (layers F.Cu F.Paste F.Mask))
  (pad G4 smd circle (at -4 -1.6) (size 0.35 0.35) (layers F.Cu F.Paste F.Mask))
  (pad F4 smd circle (at -4 -2.4) (size 0.35 0.35) (layers F.Cu F.Paste F.Mask))
  (pad E4 smd circle (at -4 -3.2) (size 0.35 0.35) (layers F.Cu F.Paste F.Mask))
  (pad D4 smd circle (at -4 -4) (size 0.35 0.35) (layers F.Cu F.Paste F.Mask) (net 6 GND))
  (pad C4 smd circle (at -4 -4.8) (size 0.35 0.35) (layers F.Cu F.Paste F.Mask))
  (pad B4 smd circle (at -4 -5.6) (size 0.35 0.35) (layers F.Cu F.Paste F.Mask))
  (pad A4 smd circle (at -4 -6.4) (size 0.35 0.35) (layers F.Cu F.Paste F.Mask))
  (pad U3 smd circle (at -4.8 6.4) (size 0.35 0.35) (layers F.Cu F.Paste F.Mask))
  (pad T3 smd circle (at -4.8 5.6) (size 0.35 0.35) (layers F.Cu F.Paste F.Mask))
  (pad R3 smd circle (at -4.8 4.8) (size 0.35 0.35) (layers F.Cu F.Paste F.Mask) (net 6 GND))
  (pad P3 smd circle (at -4.8 4) (size 0.35 0.35) (layers F.Cu F.Paste F.Mask))
  (pad N3 smd circle (at -4.8 3.2) (size 0.35 0.35) (layers F.Cu F.Paste F.Mask))
  (pad M3 smd circle (at -4.8 2.4) (size 0.35 0.35) (layers F.Cu F.Paste F.Mask))
  (pad L3 smd circle (at -4.8 1.6) (size 0.35 0.35) (layers F.Cu F.Paste F.Mask))
  (pad K3 smd circle (at -4.8 0.8) (size 0.35 0.35) (layers F.Cu F.Paste F.Mask))
  (pad J3 smd circle (at -4.8 0) (size 0.35 0.35) (layers F.Cu F.Paste F.Mask) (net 6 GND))
  (pad H3 smd circle (at -4.8 -0.8) (size 0.35 0.35) (layers F.Cu F.Paste F.Mask))
  (pad G3 smd circle (at -4.8 -1.6) (size 0.35 0.35) (layers F.Cu F.Paste F.Mask))
  (pad F3 smd circle (at -4.8 -2.4) (size 0.35 0.35) (layers F.Cu F.Paste F.Mask) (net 6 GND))
  (pad E3 smd circle (at -4.8 -3.2) (size 0.35 0.35) (layers F.Cu F.Paste F.Mask))
  (pad D3 smd circle (at -4.8 -4) (size 0.35 0.35) (layers F.Cu F.Paste F.Mask))
  (pad C3 smd circle (at -4.8 -4.8) (size 0.35 0.35) (layers F.Cu F.Paste F.Mask) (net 6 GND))
  (pad B3 smd circle (at -4.8 -5.6) (size 0.35 0.35) (layers F.Cu F.Paste F.Mask))
  (pad A3 smd circle (at -4.8 -6.4) (size 0.35 0.35) (layers F.Cu F.Paste F.Mask))
  (pad U2 smd circle (at -5.6 6.4) (size 0.35 0.35) (layers F.Cu F.Paste F.Mask))
  (pad T2 smd circle (at -5.6 5.6) (size 0.35 0.35) (layers F.Cu F.Paste F.Mask) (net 6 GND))
  (pad R2 smd circle (at -5.6 4.8) (size 0.35 0.35) (layers F.Cu F.Paste F.Mask))
  (pad P2 smd circle (at -5.6 4) (size 0.35 0.35) (layers F.Cu F.Paste F.Mask))
  (pad N2 smd circle (at -5.6 3.2) (size 0.35 0.35) (layers F.Cu F.Paste F.Mask))
  (pad L2 smd circle (at -5.6 1.6) (size 0.35 0.35) (layers F.Cu F.Paste F.Mask))
  (pad K2 smd circle (at -5.6 0.8) (size 0.35 0.35) (layers F.Cu F.Paste F.Mask))
  (pad J2 smd circle (at -5.6 0) (size 0.35 0.35) (layers F.Cu F.Paste F.Mask))
  (pad H2 smd circle (at -5.6 -0.8) (size 0.35 0.35) (layers F.Cu F.Paste F.Mask))
  (pad G2 smd circle (at -5.6 -1.6) (size 0.35 0.35) (layers F.Cu F.Paste F.Mask))
  (pad E2 smd circle (at -5.6 -3.2) (size 0.35 0.35) (layers F.Cu F.Paste F.Mask))
  (pad D2 smd circle (at -5.6 -4) (size 0.35 0.35) (layers F.Cu F.Paste F.Mask))
  (pad C2 smd circle (at -5.6 -4.8) (size 0.35 0.35) (layers F.Cu F.Paste F.Mask) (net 7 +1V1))
  (pad B2 smd circle (at -5.6 -5.6) (size 0.35 0.35) (layers F.Cu F.Paste F.Mask) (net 6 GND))
  (pad A2 smd circle (at -5.6 -6.4) (size 0.35 0.35) (layers F.Cu F.Paste F.Mask))
  (pad U1 smd circle (at -6.4 6.4) (size 0.35 0.35) (layers F.Cu F.Paste F.Mask) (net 6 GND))
  (pad T1 smd circle (at -6.4 5.6) (size 0.35 0.35) (layers F.Cu F.Paste F.Mask))
  (pad R1 smd circle (at -6.4 4.8) (size 0.35 0.35) (layers F.Cu F.Paste F.Mask))
  (pad P1 smd circle (at -6.4 4) (size 0.35 0.35) (layers F.Cu F.Paste F.Mask) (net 1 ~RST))
  (pad N1 smd circle (at -6.4 3.2) (size 0.35 0.35) (layers F.Cu F.Paste F.Mask))
  (pad L1 smd circle (at -6.4 1.6) (size 0.35 0.35) (layers F.Cu F.Paste F.Mask))
  (pad K1 smd circle (at -6.4 0.8) (size 0.35 0.35) (layers F.Cu F.Paste F.Mask))
  (pad J1 smd circle (at -6.4 0) (size 0.35 0.35) (layers F.Cu F.Paste F.Mask))
  (pad H1 smd circle (at -6.4 -0.8) (size 0.35 0.35) (layers F.Cu F.Paste F.Mask))
  (pad G1 smd circle (at -6.4 -1.6) (size 0.35 0.35) (layers F.Cu F.Paste F.Mask))
  (pad E1 smd circle (at -6.4 -3.2) (size 0.35 0.35) (layers F.Cu F.Paste F.Mask))
  (pad D1 smd circle (at -6.4 -4) (size 0.35 0.35) (layers F.Cu F.Paste F.Mask))
  (pad C1 smd circle (at -6.4 -4.8) (size 0.35 0.35) (layers F.Cu F.Paste F.Mask))
  (pad B1 smd circle (at -6.4 -5.6) (size 0.35 0.35) (layers F.Cu F.Paste F.Mask))
  (pad A1 smd circle (at -6.4 -6.4) (size 0.35 0.35) (layers F.Cu F.Paste F.Mask) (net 6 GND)))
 (gr_line (start 225 60) (end 225 230) (layer Edge.Cuts) (width 0.1))
 (gr_line (start 55 60) (end 225 60) (layer Edge.Cuts) (width 0.1))
 (gr_line (start 55 230) (end 55 60) (layer Edge.Cuts) (width 0.1))
 (gr_line (start 225 230) (end 55 230) (layer Edge.Cuts) (width 0.1))
 (segment (start 211.7 139.65) (end 211.7 139.55) (width 0.15) (layer F.Cu) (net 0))
 (segment (start 144 141) (end 144.8 140.2) (width 0.15) (layer F.Cu) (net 6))
 (segment (start 139.2 144.2) (end 140.8 144.2) (width 0.15) (layer F.Cu) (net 6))
 (segment (start 140.8 144.2) (end 140.8 145.8) (width 0.15) (layer F.Cu) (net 6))
 (segment (start 140.8 145.8) (end 139.2 145.8) (width 0.15) (layer F.Cu) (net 6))
 (segment (start 139.2 145) (end 139.2 145.8) (width 0.15) (layer F.Cu) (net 6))
 (segment (start 139.2 145) (end 140.8 145) (width 0.15) (layer F.Cu) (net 6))
 (segment (start 139.2 145) (end 139.2 144.2) (width 0.15) (layer F.Cu) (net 6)))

